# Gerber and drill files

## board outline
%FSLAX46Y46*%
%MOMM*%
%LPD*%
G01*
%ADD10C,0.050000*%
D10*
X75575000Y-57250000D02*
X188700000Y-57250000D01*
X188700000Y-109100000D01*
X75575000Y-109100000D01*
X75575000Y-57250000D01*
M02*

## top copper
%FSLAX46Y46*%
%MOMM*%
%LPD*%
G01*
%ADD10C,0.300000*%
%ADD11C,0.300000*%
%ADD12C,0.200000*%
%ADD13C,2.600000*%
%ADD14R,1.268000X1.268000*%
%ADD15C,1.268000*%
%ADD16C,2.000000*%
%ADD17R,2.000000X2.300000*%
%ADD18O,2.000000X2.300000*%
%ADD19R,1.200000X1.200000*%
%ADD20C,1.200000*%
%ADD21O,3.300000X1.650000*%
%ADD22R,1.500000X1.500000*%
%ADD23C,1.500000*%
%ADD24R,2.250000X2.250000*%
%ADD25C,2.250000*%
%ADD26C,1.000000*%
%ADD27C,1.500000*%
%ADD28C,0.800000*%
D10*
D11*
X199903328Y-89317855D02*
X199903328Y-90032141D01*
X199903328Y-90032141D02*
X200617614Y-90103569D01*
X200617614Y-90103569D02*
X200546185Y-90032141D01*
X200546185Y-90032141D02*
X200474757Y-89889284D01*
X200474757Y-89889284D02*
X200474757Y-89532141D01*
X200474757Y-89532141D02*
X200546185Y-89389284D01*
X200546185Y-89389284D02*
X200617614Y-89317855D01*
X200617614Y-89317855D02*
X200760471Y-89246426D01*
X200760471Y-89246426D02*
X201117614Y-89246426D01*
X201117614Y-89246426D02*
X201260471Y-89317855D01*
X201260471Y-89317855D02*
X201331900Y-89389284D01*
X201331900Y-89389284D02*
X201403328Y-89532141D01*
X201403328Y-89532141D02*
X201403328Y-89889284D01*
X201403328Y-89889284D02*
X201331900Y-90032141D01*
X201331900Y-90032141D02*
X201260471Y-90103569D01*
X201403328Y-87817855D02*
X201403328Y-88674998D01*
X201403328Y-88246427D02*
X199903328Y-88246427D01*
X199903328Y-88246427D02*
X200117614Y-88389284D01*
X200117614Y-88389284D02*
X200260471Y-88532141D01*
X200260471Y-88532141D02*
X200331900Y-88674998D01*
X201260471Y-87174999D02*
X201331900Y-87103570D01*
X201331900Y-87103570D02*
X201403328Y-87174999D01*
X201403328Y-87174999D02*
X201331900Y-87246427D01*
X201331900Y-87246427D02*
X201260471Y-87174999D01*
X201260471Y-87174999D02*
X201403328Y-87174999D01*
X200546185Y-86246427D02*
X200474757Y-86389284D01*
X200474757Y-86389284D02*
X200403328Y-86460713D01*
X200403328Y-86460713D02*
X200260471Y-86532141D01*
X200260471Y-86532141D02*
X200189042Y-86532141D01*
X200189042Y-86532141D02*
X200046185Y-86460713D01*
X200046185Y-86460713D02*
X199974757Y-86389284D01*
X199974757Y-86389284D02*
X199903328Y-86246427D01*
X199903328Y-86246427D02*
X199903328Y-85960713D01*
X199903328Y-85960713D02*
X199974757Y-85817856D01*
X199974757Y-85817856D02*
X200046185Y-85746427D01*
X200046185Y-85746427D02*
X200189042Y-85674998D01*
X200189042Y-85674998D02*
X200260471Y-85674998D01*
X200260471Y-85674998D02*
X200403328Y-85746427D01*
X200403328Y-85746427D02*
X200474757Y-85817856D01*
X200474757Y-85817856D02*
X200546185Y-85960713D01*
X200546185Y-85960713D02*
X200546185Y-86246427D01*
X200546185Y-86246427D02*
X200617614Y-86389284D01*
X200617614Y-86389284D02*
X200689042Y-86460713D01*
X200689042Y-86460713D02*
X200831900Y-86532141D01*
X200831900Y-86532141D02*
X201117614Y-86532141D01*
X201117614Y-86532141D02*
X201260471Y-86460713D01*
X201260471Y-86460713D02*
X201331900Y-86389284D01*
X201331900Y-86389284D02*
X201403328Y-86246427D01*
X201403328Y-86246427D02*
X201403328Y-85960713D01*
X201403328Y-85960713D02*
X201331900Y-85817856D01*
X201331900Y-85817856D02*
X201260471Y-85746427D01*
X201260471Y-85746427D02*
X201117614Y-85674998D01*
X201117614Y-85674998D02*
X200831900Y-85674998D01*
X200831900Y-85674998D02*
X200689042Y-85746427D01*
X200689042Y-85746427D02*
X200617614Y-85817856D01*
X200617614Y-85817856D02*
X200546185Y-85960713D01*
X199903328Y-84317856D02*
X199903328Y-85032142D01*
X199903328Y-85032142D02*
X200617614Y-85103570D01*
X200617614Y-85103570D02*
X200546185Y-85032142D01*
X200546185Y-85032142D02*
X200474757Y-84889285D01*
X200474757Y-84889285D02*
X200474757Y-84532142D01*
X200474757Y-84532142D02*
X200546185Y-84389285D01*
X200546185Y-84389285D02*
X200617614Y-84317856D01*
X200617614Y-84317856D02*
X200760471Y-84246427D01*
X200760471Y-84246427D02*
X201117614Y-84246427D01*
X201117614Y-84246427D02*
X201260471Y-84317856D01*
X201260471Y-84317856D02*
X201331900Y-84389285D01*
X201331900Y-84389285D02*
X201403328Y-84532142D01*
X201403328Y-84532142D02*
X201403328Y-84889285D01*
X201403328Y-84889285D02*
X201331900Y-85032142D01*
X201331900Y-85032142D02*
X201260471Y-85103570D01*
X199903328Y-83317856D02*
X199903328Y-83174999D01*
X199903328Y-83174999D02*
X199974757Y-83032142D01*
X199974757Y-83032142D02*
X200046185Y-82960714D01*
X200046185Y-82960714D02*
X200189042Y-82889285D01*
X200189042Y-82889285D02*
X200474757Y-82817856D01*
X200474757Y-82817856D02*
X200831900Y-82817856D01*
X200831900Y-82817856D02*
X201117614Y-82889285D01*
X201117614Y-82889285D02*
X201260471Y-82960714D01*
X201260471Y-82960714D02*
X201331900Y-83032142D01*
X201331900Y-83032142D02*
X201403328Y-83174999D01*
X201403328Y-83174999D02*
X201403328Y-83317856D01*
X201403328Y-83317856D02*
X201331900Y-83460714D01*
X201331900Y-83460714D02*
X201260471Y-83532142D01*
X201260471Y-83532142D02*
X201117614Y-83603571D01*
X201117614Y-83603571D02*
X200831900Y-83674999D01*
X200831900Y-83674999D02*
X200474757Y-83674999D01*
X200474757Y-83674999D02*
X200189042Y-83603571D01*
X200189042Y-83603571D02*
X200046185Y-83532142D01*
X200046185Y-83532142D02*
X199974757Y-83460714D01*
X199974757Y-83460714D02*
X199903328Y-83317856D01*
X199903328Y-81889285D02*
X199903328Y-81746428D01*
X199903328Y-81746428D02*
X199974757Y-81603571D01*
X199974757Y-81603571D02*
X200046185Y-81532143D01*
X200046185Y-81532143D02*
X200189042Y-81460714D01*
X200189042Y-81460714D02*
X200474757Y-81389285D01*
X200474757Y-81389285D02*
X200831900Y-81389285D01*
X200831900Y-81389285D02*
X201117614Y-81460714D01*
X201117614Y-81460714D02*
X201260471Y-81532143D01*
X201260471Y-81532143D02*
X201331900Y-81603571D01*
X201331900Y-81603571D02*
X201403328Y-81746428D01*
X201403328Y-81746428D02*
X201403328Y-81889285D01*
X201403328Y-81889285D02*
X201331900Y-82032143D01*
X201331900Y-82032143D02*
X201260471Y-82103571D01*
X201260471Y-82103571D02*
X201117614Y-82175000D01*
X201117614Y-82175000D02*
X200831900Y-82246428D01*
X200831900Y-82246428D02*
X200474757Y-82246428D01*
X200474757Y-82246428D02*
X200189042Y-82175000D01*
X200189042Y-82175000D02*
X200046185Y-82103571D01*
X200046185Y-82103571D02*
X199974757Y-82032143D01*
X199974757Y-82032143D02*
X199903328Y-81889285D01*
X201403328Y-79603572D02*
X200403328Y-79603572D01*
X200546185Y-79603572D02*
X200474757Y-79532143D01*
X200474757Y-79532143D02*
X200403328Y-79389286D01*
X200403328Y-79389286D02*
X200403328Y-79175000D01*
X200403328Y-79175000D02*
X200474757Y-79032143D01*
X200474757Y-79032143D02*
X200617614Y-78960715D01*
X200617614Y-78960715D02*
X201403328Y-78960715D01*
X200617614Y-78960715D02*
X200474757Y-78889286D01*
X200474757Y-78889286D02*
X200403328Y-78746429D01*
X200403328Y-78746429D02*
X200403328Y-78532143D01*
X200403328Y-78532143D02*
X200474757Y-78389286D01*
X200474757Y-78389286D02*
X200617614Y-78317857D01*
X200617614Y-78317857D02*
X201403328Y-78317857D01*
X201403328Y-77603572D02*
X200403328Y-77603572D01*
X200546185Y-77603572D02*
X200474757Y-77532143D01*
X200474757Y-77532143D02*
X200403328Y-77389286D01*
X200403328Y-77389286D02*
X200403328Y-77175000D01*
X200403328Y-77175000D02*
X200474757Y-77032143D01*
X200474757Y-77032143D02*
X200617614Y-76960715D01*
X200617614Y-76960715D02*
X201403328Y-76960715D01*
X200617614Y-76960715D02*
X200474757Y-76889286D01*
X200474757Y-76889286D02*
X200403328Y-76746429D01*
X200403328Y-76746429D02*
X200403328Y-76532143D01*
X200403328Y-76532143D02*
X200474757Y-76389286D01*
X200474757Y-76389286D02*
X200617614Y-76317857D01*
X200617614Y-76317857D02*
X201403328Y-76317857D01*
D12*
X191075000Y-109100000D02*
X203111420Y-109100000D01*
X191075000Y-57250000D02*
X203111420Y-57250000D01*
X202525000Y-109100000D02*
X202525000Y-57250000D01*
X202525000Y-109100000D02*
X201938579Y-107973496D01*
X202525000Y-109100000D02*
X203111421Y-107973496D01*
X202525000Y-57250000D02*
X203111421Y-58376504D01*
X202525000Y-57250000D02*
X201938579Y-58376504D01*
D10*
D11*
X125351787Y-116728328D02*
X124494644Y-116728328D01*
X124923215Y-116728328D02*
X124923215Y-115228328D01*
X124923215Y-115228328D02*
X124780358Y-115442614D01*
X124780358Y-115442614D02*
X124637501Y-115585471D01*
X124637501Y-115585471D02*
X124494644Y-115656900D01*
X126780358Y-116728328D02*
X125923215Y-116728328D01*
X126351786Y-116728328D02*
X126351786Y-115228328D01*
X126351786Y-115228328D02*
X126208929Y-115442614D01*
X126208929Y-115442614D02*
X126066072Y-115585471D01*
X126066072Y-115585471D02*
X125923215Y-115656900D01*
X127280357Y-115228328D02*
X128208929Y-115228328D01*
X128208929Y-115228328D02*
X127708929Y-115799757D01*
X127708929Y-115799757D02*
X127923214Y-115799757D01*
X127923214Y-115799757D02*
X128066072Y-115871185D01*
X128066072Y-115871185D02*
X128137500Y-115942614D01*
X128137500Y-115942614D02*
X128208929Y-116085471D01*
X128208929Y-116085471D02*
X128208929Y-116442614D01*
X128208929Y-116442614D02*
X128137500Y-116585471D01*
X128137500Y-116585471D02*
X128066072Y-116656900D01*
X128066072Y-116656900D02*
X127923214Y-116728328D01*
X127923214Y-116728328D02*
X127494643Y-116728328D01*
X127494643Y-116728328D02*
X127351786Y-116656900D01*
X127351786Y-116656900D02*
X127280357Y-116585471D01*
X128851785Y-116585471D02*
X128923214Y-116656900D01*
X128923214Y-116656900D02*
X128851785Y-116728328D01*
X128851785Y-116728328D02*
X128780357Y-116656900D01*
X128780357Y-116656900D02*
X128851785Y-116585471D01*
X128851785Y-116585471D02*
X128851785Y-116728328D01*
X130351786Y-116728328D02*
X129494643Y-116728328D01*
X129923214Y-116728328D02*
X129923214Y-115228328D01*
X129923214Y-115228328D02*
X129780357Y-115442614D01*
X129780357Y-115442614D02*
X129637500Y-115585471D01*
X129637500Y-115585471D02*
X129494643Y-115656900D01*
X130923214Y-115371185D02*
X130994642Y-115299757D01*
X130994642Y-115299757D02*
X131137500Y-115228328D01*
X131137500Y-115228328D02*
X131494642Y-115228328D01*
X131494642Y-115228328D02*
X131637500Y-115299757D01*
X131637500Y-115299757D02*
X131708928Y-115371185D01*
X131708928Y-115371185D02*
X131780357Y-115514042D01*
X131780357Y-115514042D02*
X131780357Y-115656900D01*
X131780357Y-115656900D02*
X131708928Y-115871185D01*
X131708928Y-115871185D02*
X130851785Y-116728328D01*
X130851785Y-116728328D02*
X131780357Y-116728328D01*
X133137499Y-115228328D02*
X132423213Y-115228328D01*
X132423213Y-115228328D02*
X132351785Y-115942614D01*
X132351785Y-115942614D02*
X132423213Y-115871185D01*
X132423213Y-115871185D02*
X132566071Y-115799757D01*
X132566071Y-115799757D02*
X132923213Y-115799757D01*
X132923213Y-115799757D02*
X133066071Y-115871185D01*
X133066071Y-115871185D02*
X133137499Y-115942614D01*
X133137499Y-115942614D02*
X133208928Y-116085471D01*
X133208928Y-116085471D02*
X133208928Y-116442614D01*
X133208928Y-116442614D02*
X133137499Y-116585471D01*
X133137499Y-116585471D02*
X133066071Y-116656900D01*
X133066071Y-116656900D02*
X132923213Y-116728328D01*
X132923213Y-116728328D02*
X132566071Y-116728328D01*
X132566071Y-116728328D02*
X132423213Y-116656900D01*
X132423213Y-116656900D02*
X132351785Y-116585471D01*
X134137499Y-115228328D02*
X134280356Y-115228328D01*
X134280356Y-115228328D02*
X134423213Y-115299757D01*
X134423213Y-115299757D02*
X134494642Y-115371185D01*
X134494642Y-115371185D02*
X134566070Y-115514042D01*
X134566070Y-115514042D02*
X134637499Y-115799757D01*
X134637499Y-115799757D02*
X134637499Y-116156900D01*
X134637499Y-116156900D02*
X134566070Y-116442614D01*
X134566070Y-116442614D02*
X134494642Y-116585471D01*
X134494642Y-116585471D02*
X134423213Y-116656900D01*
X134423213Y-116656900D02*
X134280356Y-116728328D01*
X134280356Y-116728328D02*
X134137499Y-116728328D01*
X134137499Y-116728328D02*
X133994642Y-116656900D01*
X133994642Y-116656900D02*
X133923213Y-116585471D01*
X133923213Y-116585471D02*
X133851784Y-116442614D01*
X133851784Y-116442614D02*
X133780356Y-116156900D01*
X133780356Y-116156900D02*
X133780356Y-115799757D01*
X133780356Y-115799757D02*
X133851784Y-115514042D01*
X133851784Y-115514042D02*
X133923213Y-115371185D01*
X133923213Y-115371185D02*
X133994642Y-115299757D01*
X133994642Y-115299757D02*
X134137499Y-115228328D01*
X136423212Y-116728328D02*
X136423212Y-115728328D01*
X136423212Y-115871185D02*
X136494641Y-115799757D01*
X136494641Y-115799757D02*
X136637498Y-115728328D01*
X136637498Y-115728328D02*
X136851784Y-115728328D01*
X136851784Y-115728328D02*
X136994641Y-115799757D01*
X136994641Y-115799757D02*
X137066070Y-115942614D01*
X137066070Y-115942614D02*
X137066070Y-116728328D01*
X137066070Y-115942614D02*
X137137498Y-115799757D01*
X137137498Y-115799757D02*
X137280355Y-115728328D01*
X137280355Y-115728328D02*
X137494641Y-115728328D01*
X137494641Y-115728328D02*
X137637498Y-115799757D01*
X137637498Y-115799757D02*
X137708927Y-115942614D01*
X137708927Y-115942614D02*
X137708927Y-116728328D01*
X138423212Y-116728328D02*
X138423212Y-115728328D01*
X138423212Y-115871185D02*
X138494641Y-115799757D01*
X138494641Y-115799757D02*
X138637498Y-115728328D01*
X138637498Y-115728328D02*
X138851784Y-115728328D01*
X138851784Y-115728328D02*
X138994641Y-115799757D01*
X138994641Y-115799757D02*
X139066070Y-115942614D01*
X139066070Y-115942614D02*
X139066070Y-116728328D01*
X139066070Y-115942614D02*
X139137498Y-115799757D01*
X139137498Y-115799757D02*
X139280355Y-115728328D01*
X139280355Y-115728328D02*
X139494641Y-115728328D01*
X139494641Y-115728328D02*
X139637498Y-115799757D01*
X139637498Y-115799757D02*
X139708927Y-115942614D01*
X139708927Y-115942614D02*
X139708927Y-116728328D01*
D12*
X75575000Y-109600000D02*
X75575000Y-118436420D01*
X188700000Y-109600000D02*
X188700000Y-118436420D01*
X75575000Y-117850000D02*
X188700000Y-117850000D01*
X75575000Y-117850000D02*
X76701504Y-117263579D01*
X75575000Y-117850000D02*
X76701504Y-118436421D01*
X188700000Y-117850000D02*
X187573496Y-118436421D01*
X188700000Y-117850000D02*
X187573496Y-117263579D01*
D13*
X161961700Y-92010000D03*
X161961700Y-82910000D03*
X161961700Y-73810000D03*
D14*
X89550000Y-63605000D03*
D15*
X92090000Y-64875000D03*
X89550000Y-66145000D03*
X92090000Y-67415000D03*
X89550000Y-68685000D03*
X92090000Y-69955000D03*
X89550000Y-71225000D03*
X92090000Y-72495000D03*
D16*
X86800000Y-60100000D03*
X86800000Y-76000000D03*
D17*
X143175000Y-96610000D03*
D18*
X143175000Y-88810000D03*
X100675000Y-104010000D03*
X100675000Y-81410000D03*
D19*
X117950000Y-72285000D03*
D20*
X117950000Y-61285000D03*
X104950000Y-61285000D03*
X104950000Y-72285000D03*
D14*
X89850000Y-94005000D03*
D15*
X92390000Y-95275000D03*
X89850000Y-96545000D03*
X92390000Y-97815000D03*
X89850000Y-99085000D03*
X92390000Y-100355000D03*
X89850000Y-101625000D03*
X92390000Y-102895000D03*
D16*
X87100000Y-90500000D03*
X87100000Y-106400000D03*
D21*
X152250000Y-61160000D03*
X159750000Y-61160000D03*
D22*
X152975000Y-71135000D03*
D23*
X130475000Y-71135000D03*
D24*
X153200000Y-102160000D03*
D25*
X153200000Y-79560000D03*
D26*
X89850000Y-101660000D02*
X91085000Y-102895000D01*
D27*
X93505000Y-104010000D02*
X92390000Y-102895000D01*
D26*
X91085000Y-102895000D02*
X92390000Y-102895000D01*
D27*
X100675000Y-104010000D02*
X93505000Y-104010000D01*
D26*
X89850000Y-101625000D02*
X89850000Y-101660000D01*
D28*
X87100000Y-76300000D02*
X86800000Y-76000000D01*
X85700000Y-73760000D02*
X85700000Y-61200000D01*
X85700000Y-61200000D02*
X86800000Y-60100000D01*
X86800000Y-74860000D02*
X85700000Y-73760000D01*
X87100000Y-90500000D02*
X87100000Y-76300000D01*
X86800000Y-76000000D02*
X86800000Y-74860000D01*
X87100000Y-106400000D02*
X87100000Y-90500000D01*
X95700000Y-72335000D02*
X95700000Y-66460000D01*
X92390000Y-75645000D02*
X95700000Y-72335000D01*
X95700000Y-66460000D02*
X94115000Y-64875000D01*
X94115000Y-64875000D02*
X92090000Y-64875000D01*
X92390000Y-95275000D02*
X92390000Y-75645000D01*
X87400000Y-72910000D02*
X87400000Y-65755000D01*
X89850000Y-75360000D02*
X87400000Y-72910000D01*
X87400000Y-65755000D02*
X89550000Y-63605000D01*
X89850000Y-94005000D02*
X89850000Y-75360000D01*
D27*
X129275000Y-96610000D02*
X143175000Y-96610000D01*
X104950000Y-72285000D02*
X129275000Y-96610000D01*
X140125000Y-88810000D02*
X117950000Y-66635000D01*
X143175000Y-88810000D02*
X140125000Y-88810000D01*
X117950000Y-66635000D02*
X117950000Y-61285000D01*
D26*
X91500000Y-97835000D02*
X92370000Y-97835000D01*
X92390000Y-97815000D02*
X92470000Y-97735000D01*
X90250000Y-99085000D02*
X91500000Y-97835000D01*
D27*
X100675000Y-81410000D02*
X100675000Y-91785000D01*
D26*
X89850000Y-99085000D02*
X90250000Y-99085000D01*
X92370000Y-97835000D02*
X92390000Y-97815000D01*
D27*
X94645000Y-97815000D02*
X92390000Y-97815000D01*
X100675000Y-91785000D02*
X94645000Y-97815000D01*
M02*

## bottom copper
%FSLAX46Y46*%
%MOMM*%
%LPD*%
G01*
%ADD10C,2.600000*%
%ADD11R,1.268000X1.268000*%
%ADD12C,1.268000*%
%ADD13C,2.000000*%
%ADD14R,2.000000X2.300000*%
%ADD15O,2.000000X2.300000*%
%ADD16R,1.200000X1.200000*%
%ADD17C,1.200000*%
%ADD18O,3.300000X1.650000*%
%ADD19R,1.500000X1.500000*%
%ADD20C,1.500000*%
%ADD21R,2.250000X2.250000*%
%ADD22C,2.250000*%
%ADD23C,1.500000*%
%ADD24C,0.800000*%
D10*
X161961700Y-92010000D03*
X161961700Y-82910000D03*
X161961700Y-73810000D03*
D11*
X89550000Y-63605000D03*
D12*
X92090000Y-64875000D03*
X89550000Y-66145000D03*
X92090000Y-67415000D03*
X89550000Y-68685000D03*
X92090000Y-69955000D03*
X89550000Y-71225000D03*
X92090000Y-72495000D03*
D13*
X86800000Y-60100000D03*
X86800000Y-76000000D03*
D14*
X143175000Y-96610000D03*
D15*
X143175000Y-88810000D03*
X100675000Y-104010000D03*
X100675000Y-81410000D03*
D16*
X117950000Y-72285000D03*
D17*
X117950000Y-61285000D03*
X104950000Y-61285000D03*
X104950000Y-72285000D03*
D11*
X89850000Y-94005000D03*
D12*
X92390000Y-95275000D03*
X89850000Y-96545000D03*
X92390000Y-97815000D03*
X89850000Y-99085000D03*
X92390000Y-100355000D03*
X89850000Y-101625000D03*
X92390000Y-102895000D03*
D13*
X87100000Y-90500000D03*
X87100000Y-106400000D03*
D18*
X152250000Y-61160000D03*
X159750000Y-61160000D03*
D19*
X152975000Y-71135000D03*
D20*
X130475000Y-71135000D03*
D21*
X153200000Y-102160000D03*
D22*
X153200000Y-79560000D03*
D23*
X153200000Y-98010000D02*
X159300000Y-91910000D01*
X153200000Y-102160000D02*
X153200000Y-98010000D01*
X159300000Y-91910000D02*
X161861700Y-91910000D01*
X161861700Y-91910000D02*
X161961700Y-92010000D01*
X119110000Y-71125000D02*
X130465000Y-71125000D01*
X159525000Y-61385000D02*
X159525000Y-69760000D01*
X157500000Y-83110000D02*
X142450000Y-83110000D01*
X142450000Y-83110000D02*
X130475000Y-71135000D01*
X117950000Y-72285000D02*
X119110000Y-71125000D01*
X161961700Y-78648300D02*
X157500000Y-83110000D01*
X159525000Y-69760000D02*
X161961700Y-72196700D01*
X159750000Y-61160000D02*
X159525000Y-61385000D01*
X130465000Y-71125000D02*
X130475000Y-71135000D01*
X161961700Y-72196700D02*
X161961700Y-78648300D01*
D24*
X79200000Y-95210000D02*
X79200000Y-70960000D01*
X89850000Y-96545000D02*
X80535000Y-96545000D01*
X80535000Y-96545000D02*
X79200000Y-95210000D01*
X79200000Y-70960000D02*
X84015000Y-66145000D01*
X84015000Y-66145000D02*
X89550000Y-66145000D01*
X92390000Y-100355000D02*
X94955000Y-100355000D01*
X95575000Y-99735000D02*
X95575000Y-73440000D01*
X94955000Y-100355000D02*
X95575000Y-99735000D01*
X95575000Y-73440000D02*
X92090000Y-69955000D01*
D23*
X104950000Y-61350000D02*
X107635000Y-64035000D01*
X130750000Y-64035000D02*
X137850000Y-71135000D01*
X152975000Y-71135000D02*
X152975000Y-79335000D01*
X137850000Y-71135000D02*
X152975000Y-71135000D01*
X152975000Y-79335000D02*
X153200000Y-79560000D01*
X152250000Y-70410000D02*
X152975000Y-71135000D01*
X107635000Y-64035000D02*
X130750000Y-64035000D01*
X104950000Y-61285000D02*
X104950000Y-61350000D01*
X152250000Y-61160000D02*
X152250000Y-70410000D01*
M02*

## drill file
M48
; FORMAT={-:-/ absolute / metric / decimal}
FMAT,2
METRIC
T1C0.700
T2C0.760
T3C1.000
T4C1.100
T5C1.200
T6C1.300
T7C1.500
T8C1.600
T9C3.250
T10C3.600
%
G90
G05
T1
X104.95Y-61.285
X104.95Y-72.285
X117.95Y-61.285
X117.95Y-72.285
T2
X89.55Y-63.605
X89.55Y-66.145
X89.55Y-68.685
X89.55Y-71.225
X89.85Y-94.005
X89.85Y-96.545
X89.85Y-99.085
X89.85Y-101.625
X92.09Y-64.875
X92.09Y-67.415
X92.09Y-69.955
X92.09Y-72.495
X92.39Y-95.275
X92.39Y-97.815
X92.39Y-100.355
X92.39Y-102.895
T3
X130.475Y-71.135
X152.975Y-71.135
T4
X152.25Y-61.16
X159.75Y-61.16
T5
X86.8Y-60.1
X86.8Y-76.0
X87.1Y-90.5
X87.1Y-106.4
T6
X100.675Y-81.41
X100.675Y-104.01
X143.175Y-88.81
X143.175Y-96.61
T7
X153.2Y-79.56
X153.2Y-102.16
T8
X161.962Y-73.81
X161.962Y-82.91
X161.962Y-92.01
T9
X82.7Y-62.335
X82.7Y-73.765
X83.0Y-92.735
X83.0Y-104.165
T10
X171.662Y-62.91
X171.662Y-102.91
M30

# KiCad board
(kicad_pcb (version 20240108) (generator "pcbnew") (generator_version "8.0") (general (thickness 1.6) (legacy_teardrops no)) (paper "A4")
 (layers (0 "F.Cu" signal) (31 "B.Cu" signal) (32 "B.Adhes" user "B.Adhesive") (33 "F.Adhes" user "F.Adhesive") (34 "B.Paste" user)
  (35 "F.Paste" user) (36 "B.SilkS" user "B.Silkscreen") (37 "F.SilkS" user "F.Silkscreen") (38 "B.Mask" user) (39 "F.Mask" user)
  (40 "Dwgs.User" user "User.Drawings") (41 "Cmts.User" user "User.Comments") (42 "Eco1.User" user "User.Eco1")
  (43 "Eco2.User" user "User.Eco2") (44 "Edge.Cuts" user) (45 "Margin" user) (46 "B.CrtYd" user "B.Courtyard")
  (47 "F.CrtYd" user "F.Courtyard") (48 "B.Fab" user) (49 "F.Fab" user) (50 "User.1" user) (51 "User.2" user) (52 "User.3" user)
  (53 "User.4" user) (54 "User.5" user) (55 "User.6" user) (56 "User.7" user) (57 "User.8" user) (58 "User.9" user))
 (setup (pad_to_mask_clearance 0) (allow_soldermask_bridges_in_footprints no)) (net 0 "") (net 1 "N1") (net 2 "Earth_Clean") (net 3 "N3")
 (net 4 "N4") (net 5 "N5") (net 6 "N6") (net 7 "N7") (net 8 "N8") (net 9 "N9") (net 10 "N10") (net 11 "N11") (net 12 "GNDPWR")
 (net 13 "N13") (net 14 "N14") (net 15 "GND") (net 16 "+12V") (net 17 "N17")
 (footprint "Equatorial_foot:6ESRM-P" (layer "F.Cu") (at 171.6617 82.91 90)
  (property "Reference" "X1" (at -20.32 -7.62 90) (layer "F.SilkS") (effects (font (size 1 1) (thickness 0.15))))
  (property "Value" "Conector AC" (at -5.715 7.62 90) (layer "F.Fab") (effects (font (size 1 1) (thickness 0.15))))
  (pad "" np_thru_hole circle (at -20 0 90) (size 3.6 3.6) (drill 3.6) (layers "*.Cu" "*.Mask"))
  (pad "" np_thru_hole circle (at 20 0 90) (size 3.6 3.6) (drill 3.6) (layers "*.Cu" "*.Mask"))
  (pad "1" thru_hole circle (at -9.1 -9.7 90) (size 2.6 2.6) (drill 1.6) (layers "*.Cu" "*.Mask") (remove_unused_layers no) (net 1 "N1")
   (solder_mask_margin 0.102))
  (pad "2" thru_hole circle (at 0 -9.7 90) (size 2.6 2.6) (drill 1.6) (layers "*.Cu" "*.Mask") (remove_unused_layers no)
   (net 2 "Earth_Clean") (solder_mask_margin 0.102))
  (pad "3" thru_hole circle (at 9.1 -9.7 90) (size 2.6 2.6) (drill 1.6) (layers "*.Cu" "*.Mask") (remove_unused_layers no) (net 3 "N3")
   (solder_mask_margin 0.102)))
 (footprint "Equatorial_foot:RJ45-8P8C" (layer "F.Cu") (at 83.2 68.05 -90)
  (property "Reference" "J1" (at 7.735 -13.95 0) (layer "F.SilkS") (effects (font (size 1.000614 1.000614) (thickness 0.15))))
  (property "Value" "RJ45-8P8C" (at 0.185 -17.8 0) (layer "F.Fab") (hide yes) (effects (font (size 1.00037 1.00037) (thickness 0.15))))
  (pad "" np_thru_hole circle (at -5.715 0.5 270) (size 3.25 3.25) (drill 3.25) (layers "*.Cu" "*.Mask"))
  (pad "" np_thru_hole circle (at 5.715 0.5 270) (size 3.25 3.25) (drill 3.25) (layers "*.Cu" "*.Mask"))
  (pad "1" thru_hole rect (at -4.445 -6.35 270) (size 1.268 1.268) (drill 0.76) (layers "*.Cu" "*.Mask") (remove_unused_layers no)
   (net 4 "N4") (solder_mask_margin 0.102))
  (pad "2" thru_hole circle (at -3.175 -8.89 270) (size 1.268 1.268) (drill 0.76) (layers "*.Cu" "*.Mask") (remove_unused_layers no)
   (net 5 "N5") (solder_mask_margin 0.102))
  (pad "3" thru_hole circle (at -1.905 -6.35 270) (size 1.268 1.268) (drill 0.76) (layers "*.Cu" "*.Mask") (remove_unused_layers no)
   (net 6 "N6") (solder_mask_margin 0.102))
  (pad "4" thru_hole circle (at -0.635 -8.89 270) (size 1.268 1.268) (drill 0.76) (layers "*.Cu" "*.Mask") (remove_unused_layers no)
   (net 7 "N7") (solder_mask_margin 0.102))
  (pad "5" thru_hole circle (at 0.635 -6.35 270) (size 1.268 1.268) (drill 0.76) (layers "*.Cu" "*.Mask") (remove_unused_layers no)
   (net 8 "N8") (solder_mask_margin 0.102))
  (pad "6" thru_hole circle (at 1.905 -8.89 270) (size 1.268 1.268) (drill 0.76) (layers "*.Cu" "*.Mask") (remove_unused_layers no)
   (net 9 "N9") (solder_mask_margin 0.102))
  (pad "7" thru_hole circle (at 3.175 -6.35 270) (size 1.268 1.268) (drill 0.76) (layers "*.Cu" "*.Mask") (remove_unused_layers no)
   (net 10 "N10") (solder_mask_margin 0.102))
  (pad "8" thru_hole circle (at 4.445 -8.89 270) (size 1.268 1.268) (drill 0.76) (layers "*.Cu" "*.Mask") (remove_unused_layers no)
   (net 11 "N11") (solder_mask_margin 0.102))
  (pad "9" thru_hole circle (at -7.95 -3.6 270) (size 2 2) (drill 1.2) (layers "*.Cu" "*.Mask") (remove_unused_layers no) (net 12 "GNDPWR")
   (solder_mask_margin 0.102))
  (pad "10" thru_hole circle (at 7.95 -3.6 270) (size 2 2) (drill 1.2) (layers "*.Cu" "*.Mask") (remove_unused_layers no) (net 12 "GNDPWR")
   (solder_mask_margin 0.102)))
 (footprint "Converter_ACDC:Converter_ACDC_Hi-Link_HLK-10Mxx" (layer "F.Cu") (at 143.175 96.61 180)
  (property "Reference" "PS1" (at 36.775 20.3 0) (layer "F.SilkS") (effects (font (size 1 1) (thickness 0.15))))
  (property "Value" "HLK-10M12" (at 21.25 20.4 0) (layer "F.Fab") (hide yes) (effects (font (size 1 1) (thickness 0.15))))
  (pad "1" thru_hole rect (at 0 0 180) (size 2 2.3) (drill 1.3) (layers "*.Cu" "*.Mask") (remove_unused_layers no) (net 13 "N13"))
  (pad "2" thru_hole oval (at 0 7.8 180) (size 2 2.3) (drill 1.3) (layers "*.Cu" "*.Mask") (remove_unused_layers no) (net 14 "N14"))
  (pad "3" thru_hole oval (at 42.5 -7.4 180) (size 2 2.3) (drill 1.3) (layers "*.Cu" "*.Mask") (remove_unused_layers no) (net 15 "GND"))
  (pad "4" thru_hole oval (at 42.5 15.2 180) (size 2 2.3) (drill 1.3) (layers "*.Cu" "*.Mask") (remove_unused_layers no) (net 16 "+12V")))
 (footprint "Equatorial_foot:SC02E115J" (layer "F.Cu") (at 117.95 72.285 180)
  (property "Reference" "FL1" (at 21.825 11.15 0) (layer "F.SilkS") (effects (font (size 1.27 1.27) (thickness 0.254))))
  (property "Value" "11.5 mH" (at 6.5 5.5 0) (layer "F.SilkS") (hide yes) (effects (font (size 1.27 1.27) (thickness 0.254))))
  (pad "1" thru_hole rect (at 0 0 180) (size 1.2 1.2) (drill 0.7) (layers "*.Cu" "*.Mask") (remove_unused_layers no) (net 3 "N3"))
  (pad "2" thru_hole circle (at 0 11 180) (size 1.2 1.2) (drill 0.7) (layers "*.Cu" "*.Mask") (remove_unused_layers no) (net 14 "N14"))
  (pad "3" thru_hole circle (at 13 11 180) (size 1.2 1.2) (drill 0.7) (layers "*.Cu" "*.Mask") (remove_unused_layers no) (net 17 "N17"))
  (pad "4" thru_hole circle (at 13 0 180) (size 1.2 1.2) (drill 0.7) (layers "*.Cu" "*.Mask") (remove_unused_layers no) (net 13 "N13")))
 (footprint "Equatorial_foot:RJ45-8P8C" (layer "F.Cu") (at 83.5 98.45 -90)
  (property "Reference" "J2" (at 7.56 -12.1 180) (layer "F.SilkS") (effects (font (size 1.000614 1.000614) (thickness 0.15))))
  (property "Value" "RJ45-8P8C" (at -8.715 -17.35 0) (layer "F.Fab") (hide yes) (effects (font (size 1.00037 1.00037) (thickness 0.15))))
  (pad "" np_thru_hole circle (at -5.715 0.5 270) (size 3.25 3.25) (drill 3.25) (layers "*.Cu" "*.Mask"))
  (pad "" np_thru_hole circle (at 5.715 0.5 270) (size 3.25 3.25) (drill 3.25) (layers "*.Cu" "*.Mask"))
  (pad "1" thru_hole rect (at -4.445 -6.35 270) (size 1.268 1.268) (drill 0.76) (layers "*.Cu" "*.Mask") (remove_unused_layers no)
   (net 4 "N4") (solder_mask_margin 0.102))
  (pad "2" thru_hole circle (at -3.175 -8.89 270) (size 1.268 1.268) (drill 0.76) (layers "*.Cu" "*.Mask") (remove_unused_layers no)
   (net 5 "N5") (solder_mask_margin 0.102))
  (pad "3" thru_hole circle (at -1.905 -6.35 270) (size 1.268 1.268) (drill 0.76) (layers "*.Cu" "*.Mask") (remove_unused_layers no)
   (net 6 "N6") (solder_mask_margin 0.102))
  (pad "4" thru_hole circle (at -0.635 -8.89 270) (size 1.268 1.268) (drill 0.76) (layers "*.Cu" "*.Mask") (remove_unused_layers no)
   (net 16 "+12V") (solder_mask_margin 0.102))
  (pad "5" thru_hole circle (at 0.635 -6.35 270) (size 1.268 1.268) (drill 0.76) (layers "*.Cu" "*.Mask") (remove_unused_layers no)
   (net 16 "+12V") (solder_mask_margin 0.102))
  (pad "6" thru_hole circle (at 1.905 -8.89 270) (size 1.268 1.268) (drill 0.76) (layers "*.Cu" "*.Mask") (remove_unused_layers no)
   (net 9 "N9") (solder_mask_margin 0.102))
  (pad "7" thru_hole circle (at 3.175 -6.35 270) (size 1.268 1.268) (drill 0.76) (layers "*.Cu" "*.Mask") (remove_unused_layers no)
   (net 15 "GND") (solder_mask_margin 0.102))
  (pad "8" thru_hole circle (at 4.445 -8.89 270) (size 1.268 1.268) (drill 0.76) (layers "*.Cu" "*.Mask") (remove_unused_layers no)
   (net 15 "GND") (solder_mask_margin 0.102))
  (pad "9" thru_hole circle (at -7.95 -3.6 270) (size 2 2) (drill 1.2) (layers "*.Cu" "*.Mask") (remove_unused_layers no) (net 12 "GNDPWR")
   (solder_mask_margin 0.102))
  (pad "10" thru_hole circle (at 7.95 -3.6 270) (size 2 2) (drill 1.2) (layers "*.Cu" "*.Mask") (remove_unused_layers no) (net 12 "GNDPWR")
   (solder_mask_margin 0.102)))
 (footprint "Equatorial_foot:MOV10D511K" (layer "F.Cu") (at 152.25 61.16)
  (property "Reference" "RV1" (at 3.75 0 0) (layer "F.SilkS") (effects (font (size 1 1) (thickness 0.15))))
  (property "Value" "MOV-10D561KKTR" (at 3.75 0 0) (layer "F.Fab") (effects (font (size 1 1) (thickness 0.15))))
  (pad "1" thru_hole oval (at 0 0) (size 3.3 1.65) (drill 1.1) (layers "*.Cu" "*.Mask") (remove_unused_layers no) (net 17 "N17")
   (solder_mask_margin 0.102))
  (pad "2" thru_hole oval (at 7.5 0) (size 3.3 1.65) (drill 1.1) (layers "*.Cu" "*.Mask") (remove_unused_layers no) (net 3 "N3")
   (solder_mask_margin 0.102)))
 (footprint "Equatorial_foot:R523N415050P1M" (layer "F.Cu") (at 152.975 71.135 180)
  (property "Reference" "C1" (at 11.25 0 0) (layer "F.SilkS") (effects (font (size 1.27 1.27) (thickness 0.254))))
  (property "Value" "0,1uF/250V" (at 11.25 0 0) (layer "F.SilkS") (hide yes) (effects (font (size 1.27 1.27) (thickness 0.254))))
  (pad "1" thru_hole rect (at 0 0 180) (size 1.5 1.5) (drill 1) (layers "*.Cu" "*.Mask") (remove_unused_layers no) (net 17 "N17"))
  (pad "2" thru_hole circle (at 22.5 0 180) (size 1.5 1.5) (drill 1) (layers "*.Cu" "*.Mask") (remove_unused_layers no) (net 3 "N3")))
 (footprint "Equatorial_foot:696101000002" (layer "F.Cu") (at 153.2 102.16 90)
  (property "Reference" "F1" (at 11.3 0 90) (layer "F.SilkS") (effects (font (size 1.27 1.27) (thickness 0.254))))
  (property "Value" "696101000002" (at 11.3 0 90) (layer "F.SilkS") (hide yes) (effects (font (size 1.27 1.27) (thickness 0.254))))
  (pad "1" thru_hole rect (at 0 0 90) (size 2.25 2.25) (drill 1.5) (layers "*.Cu" "*.Mask") (remove_unused_layers no) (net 1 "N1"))
  (pad "2" thru_hole circle (at 22.6 0 90) (size 2.25 2.25) (drill 1.5) (layers "*.Cu" "*.Mask") (remove_unused_layers no) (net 17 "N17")))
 (gr_rect (start 75.575 57.25) (end 188.7 109.1) (stroke (width 0.05) (type default)) (fill none) (layer "Edge.Cuts"))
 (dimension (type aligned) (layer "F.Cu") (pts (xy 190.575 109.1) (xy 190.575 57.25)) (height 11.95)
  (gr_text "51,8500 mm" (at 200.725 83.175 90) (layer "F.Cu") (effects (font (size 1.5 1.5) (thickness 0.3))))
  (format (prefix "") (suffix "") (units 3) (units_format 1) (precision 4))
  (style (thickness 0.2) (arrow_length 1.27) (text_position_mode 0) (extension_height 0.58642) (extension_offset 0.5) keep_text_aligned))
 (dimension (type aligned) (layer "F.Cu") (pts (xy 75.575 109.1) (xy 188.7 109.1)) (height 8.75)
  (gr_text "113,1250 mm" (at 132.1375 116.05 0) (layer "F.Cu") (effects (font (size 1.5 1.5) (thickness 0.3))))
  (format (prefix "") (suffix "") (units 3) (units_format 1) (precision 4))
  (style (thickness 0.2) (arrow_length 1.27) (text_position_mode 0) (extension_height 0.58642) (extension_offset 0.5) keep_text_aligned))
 (segment (start 153.2 98.01) (end 159.3 91.91) (width 1.5) (layer "B.Cu") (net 1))
 (segment (start 153.2 102.16) (end 153.2 98.01) (width 1.5) (layer "B.Cu") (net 1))
 (segment (start 159.3 91.91) (end 161.8617 91.91) (width 1.5) (layer "B.Cu") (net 1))
 (segment (start 161.8617 91.91) (end 161.9617 92.01) (width 1.5) (layer "B.Cu") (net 1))
 (segment (start 89.85 101.66) (end 91.085 102.895) (width 1) (layer "F.Cu") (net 15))
 (segment (start 93.505 104.01) (end 92.39 102.895) (width 1.5) (layer "F.Cu") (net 15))
 (segment (start 91.085 102.895) (end 92.39 102.895) (width 1) (layer "F.Cu") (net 15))
 (segment (start 100.675 104.01) (end 93.505 104.01) (width 1.5) (layer "F.Cu") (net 15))
 (segment (start 89.85 101.625) (end 89.85 101.66) (width 1) (layer "F.Cu") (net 15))
 (segment (start 119.11 71.125) (end 130.465 71.125) (width 1.5) (layer "B.Cu") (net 3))
 (segment (start 159.525 61.385) (end 159.525 69.76) (width 1.5) (layer "B.Cu") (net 3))
 (segment (start 157.5 83.11) (end 142.45 83.11) (width 1.5) (layer "B.Cu") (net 3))
 (segment (start 142.45 83.11) (end 130.475 71.135) (width 1.5) (layer "B.Cu") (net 3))
 (segment (start 117.95 72.285) (end 119.11 71.125) (width 1.5) (layer "B.Cu") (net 3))
 (segment (start 161.9617 78.6483) (end 157.5 83.11) (width 1.5) (layer "B.Cu") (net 3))
 (segment (start 159.525 69.76) (end 161.9617 72.1967) (width 1.5) (layer "B.Cu") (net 3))
 (segment (start 159.75 61.16) (end 159.525 61.385) (width 1.5) (layer "B.Cu") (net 3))
 (segment (start 130.465 71.125) (end 130.475 71.135) (width 1.5) (layer "B.Cu") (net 3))
 (segment (start 161.9617 72.1967) (end 161.9617 78.6483) (width 1.5) (layer "B.Cu") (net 3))
 (segment (start 87.1 76.3) (end 86.8 76) (width 0.8) (layer "F.Cu") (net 12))
 (segment (start 85.7 73.76) (end 85.7 61.2) (width 0.8) (layer "F.Cu") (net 12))
 (segment (start 85.7 61.2) (end 86.8 60.1) (width 0.8) (layer "F.Cu") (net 12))
 (segment (start 86.8 74.86) (end 85.7 73.76) (width 0.8) (layer "F.Cu") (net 12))
 (segment (start 87.1 90.5) (end 87.1 76.3) (width 0.8) (layer "F.Cu") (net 12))
 (segment (start 86.8 76) (end 86.8 74.86) (width 0.8) (layer "F.Cu") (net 12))
 (segment (start 87.1 106.4) (end 87.1 90.5) (width 0.8) (layer "F.Cu") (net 12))
 (segment (start 95.7 72.335) (end 95.7 66.46) (width 0.8) (layer "F.Cu") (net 5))
 (segment (start 92.39 75.645) (end 95.7 72.335) (width 0.8) (layer "F.Cu") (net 5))
 (segment (start 95.7 66.46) (end 94.115 64.875) (width 0.8) (layer "F.Cu") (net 5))
 (segment (start 94.115 64.875) (end 92.09 64.875) (width 0.8) (layer "F.Cu") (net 5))
 (segment (start 92.39 95.275) (end 92.39 75.645) (width 0.8) (layer "F.Cu") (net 5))
 (segment (start 79.2 95.21) (end 79.2 70.96) (width 0.8) (layer "B.Cu") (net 6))
 (segment (start 89.85 96.545) (end 80.535 96.545) (width 0.8) (layer "B.Cu") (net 6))
 (segment (start 80.535 96.545) (end 79.2 95.21) (width 0.8) (layer "B.Cu") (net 6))
 (segment (start 79.2 70.96) (end 84.015 66.145) (width 0.8) (layer "B.Cu") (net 6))
 (segment (start 84.015 66.145) (end 89.55 66.145) (width 0.8) (layer "B.Cu") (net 6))
 (segment (start 92.39 100.355) (end 94.955 100.355) (width 0.8) (layer "B.Cu") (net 9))
 (segment (start 95.575 99.735) (end 95.575 73.44) (width 0.8) (layer "B.Cu") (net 9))
 (segment (start 94.955 100.355) (end 95.575 99.735) (width 0.8) (layer "B.Cu") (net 9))
 (segment (start 95.575 73.44) (end 92.09 69.955) (width 0.8) (layer "B.Cu") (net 9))
 (segment (start 87.4 72.91) (end 87.4 65.755) (width 0.8) (layer "F.Cu") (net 4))
 (segment (start 89.85 75.36) (end 87.4 72.91) (width 0.8) (layer "F.Cu") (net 4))
 (segment (start 87.4 65.755) (end 89.55 63.605) (width 0.8) (layer "F.Cu") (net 4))
 (segment (start 89.85 94.005) (end 89.85 75.36) (width 0.8) (layer "F.Cu") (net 4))
 (segment (start 104.95 61.35) (end 107.635 64.035) (width 1.5) (layer "B.Cu") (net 17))
 (segment (start 130.75 64.035) (end 137.85 71.135) (width 1.5) (layer "B.Cu") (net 17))
 (segment (start 152.975 71.135) (end 152.975 79.335) (width 1.5) (layer "B.Cu") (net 17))
 (segment (start 137.85 71.135) (end 152.975 71.135) (width 1.5) (layer "B.Cu") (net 17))
 (segment (start 152.975 79.335) (end 153.2 79.56) (width 1.5) (layer "B.Cu") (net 17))
 (segment (start 152.25 70.41) (end 152.975 71.135) (width 1.5) (layer "B.Cu") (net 17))
 (segment (start 107.635 64.035) (end 130.75 64.035) (width 1.5) (layer "B.Cu") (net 17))
 (segment (start 104.95 61.285) (end 104.95 61.35) (width 1.5) (layer "B.Cu") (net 17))
 (segment (start 152.25 61.16) (end 152.25 70.41) (width 1.5) (layer "B.Cu") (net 17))
 (segment (start 129.275 96.61) (end 143.175 96.61) (width 1.5) (layer "F.Cu") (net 13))
 (segment (start 104.95 72.285) (end 129.275 96.61) (width 1.5) (layer "F.Cu") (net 13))
 (segment (start 140.125 88.81) (end 117.95 66.635) (width 1.5) (layer "F.Cu") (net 14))
 (segment (start 143.175 88.81) (end 140.125 88.81) (width 1.5) (layer "F.Cu") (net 14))
 (segment (start 117.95 66.635) (end 117.95 61.285) (width 1.5) (layer "F.Cu") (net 14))
 (segment (start 91.5 97.835) (end 92.37 97.835) (width 1) (layer "F.Cu") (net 16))
 (segment (start 92.39 97.815) (end 92.47 97.735) (width 1) (layer "F.Cu") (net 16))
 (segment (start 90.25 99.085) (end 91.5 97.835) (width 1) (layer "F.Cu") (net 16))
 (segment (start 100.675 81.41) (end 100.675 91.785) (width 1.5) (layer "F.Cu") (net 16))
 (segment (start 89.85 99.085) (end 90.25 99.085) (width 1) (layer "F.Cu") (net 16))
 (segment (start 92.37 97.835) (end 92.39 97.815) (width 1) (layer "F.Cu") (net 16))
 (segment (start 94.645 97.815) (end 92.39 97.815) (width 1.5) (layer "F.Cu") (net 16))
 (segment (start 100.675 91.785) (end 94.645 97.815) (width 1.5) (layer "F.Cu") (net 16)))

